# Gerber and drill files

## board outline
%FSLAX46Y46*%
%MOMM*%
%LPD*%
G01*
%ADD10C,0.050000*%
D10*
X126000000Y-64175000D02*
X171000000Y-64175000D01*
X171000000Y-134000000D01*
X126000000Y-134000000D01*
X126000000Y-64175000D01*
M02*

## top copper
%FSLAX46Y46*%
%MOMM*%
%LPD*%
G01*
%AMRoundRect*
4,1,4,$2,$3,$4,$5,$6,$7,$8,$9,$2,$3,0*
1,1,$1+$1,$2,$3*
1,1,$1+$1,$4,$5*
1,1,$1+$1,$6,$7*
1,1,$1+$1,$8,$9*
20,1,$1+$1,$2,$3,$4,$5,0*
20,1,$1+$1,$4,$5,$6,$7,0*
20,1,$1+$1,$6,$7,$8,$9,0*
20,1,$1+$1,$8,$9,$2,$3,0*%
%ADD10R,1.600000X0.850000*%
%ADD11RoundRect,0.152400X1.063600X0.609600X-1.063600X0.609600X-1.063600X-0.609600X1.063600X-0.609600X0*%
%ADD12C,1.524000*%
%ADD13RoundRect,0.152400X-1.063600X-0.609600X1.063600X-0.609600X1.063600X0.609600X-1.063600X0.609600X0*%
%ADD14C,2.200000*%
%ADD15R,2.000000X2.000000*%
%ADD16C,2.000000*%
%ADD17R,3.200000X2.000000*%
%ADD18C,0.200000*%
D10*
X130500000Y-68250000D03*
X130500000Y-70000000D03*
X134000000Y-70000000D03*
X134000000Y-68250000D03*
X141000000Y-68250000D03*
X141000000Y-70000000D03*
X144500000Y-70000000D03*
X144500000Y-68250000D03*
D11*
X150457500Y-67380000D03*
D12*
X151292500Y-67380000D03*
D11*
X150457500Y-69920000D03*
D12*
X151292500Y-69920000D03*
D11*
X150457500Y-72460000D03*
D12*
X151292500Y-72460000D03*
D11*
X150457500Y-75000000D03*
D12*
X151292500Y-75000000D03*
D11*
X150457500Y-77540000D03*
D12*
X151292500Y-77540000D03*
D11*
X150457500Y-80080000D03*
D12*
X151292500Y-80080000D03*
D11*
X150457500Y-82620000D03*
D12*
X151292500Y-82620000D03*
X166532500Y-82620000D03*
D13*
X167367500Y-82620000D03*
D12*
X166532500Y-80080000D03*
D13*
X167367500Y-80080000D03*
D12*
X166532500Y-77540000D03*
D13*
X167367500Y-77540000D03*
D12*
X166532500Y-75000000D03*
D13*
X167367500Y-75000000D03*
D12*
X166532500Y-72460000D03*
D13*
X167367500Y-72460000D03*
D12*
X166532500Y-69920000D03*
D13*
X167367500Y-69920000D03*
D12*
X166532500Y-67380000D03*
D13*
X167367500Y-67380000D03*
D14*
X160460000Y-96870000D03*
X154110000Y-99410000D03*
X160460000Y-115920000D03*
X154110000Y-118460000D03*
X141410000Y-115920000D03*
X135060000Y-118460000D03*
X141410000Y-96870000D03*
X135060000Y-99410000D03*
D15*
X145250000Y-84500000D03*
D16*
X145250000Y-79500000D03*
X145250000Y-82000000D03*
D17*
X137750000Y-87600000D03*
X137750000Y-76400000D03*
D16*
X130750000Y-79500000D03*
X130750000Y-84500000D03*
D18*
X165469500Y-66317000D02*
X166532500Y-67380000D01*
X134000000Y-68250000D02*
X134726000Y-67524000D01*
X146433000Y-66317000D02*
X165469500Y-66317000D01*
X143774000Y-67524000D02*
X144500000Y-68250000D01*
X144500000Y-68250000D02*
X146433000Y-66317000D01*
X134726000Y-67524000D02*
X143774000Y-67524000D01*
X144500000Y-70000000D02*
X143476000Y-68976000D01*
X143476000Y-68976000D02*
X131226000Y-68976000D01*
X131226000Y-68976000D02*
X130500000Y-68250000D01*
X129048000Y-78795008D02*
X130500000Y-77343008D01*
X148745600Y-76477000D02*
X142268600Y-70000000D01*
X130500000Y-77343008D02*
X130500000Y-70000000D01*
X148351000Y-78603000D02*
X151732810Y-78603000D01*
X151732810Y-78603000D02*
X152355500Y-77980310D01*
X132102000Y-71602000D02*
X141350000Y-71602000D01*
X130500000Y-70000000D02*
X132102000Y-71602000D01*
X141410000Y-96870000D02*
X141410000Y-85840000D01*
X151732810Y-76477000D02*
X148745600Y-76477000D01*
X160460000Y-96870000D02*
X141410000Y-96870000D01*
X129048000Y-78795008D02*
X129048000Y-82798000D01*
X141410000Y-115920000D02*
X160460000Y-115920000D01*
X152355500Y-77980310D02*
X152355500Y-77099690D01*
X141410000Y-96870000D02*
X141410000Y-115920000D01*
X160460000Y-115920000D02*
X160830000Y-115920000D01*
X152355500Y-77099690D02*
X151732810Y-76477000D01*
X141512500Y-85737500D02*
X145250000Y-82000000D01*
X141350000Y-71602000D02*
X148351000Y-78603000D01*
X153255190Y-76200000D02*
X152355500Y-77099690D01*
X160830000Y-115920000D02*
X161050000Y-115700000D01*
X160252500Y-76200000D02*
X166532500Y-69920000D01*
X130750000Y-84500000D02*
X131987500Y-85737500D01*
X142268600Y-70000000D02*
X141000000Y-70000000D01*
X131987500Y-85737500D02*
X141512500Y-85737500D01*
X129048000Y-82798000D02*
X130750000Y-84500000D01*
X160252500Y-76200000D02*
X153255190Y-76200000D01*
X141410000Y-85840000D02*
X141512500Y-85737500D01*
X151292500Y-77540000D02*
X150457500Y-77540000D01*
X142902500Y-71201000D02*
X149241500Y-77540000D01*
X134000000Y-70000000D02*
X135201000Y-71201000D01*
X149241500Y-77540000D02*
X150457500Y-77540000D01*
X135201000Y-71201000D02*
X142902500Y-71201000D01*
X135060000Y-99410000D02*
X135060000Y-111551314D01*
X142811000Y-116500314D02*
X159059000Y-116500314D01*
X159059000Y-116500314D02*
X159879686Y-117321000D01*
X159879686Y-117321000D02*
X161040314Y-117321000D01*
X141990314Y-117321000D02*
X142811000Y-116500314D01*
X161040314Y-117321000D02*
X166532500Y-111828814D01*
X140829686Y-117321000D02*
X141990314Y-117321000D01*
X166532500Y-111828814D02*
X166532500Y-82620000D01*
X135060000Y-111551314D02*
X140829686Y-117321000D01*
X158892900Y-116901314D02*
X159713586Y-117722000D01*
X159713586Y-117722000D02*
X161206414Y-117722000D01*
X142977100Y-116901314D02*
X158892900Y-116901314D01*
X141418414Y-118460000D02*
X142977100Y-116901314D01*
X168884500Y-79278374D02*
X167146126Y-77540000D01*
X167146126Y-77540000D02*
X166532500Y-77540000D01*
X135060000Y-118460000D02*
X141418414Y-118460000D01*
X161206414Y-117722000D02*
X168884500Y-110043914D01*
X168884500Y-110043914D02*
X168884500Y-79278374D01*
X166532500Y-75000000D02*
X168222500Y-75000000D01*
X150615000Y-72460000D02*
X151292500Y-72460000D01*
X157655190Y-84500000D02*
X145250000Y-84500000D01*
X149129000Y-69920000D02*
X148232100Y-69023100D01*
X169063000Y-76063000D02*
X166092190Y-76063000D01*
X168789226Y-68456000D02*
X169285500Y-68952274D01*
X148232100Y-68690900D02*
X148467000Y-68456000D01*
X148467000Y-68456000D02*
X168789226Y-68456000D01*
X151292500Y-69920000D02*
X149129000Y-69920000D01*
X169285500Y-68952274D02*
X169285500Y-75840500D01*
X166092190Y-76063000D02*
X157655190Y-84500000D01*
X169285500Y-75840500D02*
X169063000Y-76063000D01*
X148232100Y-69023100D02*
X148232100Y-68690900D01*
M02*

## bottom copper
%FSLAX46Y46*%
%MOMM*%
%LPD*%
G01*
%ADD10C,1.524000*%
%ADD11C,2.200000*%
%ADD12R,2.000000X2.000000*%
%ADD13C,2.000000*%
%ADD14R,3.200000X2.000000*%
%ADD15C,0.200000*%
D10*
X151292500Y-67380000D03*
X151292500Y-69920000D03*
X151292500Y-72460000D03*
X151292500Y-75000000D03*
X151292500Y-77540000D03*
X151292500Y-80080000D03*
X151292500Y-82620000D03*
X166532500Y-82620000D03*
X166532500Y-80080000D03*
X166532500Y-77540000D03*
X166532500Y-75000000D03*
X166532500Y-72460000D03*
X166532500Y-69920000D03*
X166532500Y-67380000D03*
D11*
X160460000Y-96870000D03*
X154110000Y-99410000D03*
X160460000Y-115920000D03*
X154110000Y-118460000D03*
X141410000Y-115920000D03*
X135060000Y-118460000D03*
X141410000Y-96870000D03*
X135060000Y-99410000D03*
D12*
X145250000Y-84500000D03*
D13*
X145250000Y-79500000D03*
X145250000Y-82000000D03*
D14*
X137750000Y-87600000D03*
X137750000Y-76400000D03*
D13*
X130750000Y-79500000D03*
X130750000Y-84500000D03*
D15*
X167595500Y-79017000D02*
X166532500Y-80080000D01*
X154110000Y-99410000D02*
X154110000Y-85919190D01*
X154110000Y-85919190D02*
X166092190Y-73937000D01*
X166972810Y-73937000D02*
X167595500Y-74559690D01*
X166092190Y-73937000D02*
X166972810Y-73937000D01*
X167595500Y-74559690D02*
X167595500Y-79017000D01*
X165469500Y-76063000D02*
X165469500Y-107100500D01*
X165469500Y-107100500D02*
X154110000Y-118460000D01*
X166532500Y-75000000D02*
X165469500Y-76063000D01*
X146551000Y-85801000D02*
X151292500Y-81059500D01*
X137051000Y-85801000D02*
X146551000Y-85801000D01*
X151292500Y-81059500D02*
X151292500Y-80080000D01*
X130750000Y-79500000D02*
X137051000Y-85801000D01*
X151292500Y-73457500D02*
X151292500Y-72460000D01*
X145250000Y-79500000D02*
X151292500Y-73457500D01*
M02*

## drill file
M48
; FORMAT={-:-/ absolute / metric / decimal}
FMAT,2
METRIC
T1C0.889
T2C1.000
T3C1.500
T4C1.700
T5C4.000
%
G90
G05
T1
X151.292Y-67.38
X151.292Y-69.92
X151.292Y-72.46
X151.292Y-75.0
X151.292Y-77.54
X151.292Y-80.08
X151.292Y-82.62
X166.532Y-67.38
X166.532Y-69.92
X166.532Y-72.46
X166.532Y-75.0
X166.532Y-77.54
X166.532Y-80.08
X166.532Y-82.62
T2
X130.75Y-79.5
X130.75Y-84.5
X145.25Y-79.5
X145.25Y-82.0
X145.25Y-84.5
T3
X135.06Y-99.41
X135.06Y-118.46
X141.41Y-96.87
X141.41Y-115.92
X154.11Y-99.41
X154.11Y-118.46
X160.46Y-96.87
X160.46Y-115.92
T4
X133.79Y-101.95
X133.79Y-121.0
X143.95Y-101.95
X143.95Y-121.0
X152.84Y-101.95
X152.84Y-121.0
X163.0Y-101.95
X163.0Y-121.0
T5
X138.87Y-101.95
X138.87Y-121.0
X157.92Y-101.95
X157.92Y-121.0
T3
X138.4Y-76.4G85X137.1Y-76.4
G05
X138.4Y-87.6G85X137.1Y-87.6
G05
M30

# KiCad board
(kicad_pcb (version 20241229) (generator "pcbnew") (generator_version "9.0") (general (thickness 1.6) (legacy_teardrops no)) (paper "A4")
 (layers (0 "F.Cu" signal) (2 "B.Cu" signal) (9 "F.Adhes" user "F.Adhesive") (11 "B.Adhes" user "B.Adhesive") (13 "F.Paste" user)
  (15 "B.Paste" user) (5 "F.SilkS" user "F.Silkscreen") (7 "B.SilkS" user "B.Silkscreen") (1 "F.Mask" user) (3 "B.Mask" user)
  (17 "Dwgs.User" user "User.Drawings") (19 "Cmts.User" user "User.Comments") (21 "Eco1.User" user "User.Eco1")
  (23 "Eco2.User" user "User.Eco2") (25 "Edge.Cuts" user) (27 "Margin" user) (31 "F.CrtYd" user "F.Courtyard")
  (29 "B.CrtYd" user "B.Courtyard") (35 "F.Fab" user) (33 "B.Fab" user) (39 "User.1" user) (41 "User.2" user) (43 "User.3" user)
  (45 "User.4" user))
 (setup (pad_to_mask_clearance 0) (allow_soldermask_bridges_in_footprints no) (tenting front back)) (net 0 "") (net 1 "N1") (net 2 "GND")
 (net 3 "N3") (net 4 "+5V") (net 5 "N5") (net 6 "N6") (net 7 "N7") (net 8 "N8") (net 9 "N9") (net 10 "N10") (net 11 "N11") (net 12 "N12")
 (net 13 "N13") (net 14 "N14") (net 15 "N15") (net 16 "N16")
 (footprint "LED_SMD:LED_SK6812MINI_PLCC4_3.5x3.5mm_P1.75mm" (layer "F.Cu") (at 132.25 69.125)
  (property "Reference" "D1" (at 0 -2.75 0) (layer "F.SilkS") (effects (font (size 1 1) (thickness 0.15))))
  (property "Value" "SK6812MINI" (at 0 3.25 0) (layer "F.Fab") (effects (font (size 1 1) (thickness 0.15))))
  (pad "1" smd rect (at -1.75 -0.875) (size 1.6 0.85) (layers "F.Cu" "F.Mask" "F.Paste") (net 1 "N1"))
  (pad "2" smd rect (at -1.75 0.875) (size 1.6 0.85) (layers "F.Cu" "F.Mask" "F.Paste") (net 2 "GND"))
  (pad "3" smd rect (at 1.75 0.875) (size 1.6 0.85) (layers "F.Cu" "F.Mask" "F.Paste") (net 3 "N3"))
  (pad "4" smd rect (at 1.75 -0.875) (size 1.6 0.85) (layers "F.Cu" "F.Mask" "F.Paste") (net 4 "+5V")))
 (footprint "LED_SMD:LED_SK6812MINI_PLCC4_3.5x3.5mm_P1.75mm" (layer "F.Cu") (at 142.75 69.125)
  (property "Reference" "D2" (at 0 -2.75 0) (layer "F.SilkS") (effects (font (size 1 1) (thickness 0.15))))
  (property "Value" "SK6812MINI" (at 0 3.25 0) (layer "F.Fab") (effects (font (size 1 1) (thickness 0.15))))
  (pad "1" smd rect (at -1.75 -0.875) (size 1.6 0.85) (layers "F.Cu" "F.Mask" "F.Paste") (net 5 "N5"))
  (pad "2" smd rect (at -1.75 0.875) (size 1.6 0.85) (layers "F.Cu" "F.Mask" "F.Paste") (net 2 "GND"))
  (pad "3" smd rect (at 1.75 0.875) (size 1.6 0.85) (layers "F.Cu" "F.Mask" "F.Paste") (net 1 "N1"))
  (pad "4" smd rect (at 1.75 -0.875) (size 1.6 0.85) (layers "F.Cu" "F.Mask" "F.Paste") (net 4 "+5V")))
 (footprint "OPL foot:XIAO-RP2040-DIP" (layer "F.Cu") (at 158.9125 75)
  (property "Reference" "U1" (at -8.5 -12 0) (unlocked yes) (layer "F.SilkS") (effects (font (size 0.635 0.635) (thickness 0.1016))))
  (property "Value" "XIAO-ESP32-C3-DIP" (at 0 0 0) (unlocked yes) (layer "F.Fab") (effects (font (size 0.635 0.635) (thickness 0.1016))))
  (pad "1" smd roundrect (at -8.455 -7.62 180) (size 2.432 1.524) (layers "F.Cu" "F.Mask") (roundrect_rratio 0.1) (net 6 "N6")
   (thermal_bridge_angle 45))
  (pad "1" thru_hole circle (at -7.62 -7.62 180) (size 1.524 1.524) (drill 0.889) (layers "*.Cu" "*.Mask") (remove_unused_layers no)
   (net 6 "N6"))
  (pad "2" smd roundrect (at -8.455 -5.08 180) (size 2.432 1.524) (layers "F.Cu" "F.Mask") (roundrect_rratio 0.1) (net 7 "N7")
   (thermal_bridge_angle 45))
  (pad "2" thru_hole circle (at -7.62 -5.08 180) (size 1.524 1.524) (drill 0.889) (layers "*.Cu" "*.Mask") (remove_unused_layers no)
   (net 7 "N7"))
  (pad "3" smd roundrect (at -8.455 -2.54 180) (size 2.432 1.524) (layers "F.Cu" "F.Mask") (roundrect_rratio 0.1) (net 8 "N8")
   (thermal_bridge_angle 45))
  (pad "3" thru_hole circle (at -7.62 -2.54 180) (size 1.524 1.524) (drill 0.889) (layers "*.Cu" "*.Mask") (remove_unused_layers no)
   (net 8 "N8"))
  (pad "4" smd roundrect (at -8.455 0 180) (size 2.432 1.524) (layers "F.Cu" "F.Mask") (roundrect_rratio 0.1) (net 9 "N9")
   (thermal_bridge_angle 45))
  (pad "4" thru_hole circle (at -7.62 0 180) (size 1.524 1.524) (drill 0.889) (layers "*.Cu" "*.Mask") (remove_unused_layers no)
   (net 9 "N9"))
  (pad "5" smd roundrect (at -8.455 2.54 180) (size 2.432 1.524) (layers "F.Cu" "F.Mask") (roundrect_rratio 0.1) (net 3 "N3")
   (thermal_bridge_angle 45))
  (pad "5" thru_hole circle (at -7.62 2.54 180) (size 1.524 1.524) (drill 0.889) (layers "*.Cu" "*.Mask") (remove_unused_layers no)
   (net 3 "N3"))
  (pad "6" smd roundrect (at -8.455 5.08 180) (size 2.432 1.524) (layers "F.Cu" "F.Mask") (roundrect_rratio 0.1) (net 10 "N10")
   (thermal_bridge_angle 45))
  (pad "6" thru_hole circle (at -7.62 5.08 180) (size 1.524 1.524) (drill 0.889) (layers "*.Cu" "*.Mask") (remove_unused_layers no)
   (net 10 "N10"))
  (pad "7" smd roundrect (at -8.455 7.62 180) (size 2.432 1.524) (layers "F.Cu" "F.Mask") (roundrect_rratio 0.1) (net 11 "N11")
   (thermal_bridge_angle 45))
  (pad "7" thru_hole circle (at -7.62 7.62 180) (size 1.524 1.524) (drill 0.889) (layers "*.Cu" "*.Mask") (remove_unused_layers no)
   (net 11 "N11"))
  (pad "8" thru_hole circle (at 7.62 7.62) (size 1.524 1.524) (drill 0.889) (layers "*.Cu" "*.Mask") (remove_unused_layers no)
   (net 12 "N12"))
  (pad "8" smd roundrect (at 8.455 7.62) (size 2.432 1.524) (layers "F.Cu" "F.Mask") (roundrect_rratio 0.1) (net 12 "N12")
   (thermal_bridge_angle 45))
  (pad "9" thru_hole circle (at 7.62 5.08) (size 1.524 1.524) (drill 0.889) (layers "*.Cu" "*.Mask") (remove_unused_layers no)
   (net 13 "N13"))
  (pad "9" smd roundrect (at 8.455 5.08) (size 2.432 1.524) (layers "F.Cu" "F.Mask") (roundrect_rratio 0.1) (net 13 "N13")
   (thermal_bridge_angle 45))
  (pad "10" thru_hole circle (at 7.62 2.54) (size 1.524 1.524) (drill 0.889) (layers "*.Cu" "*.Mask") (remove_unused_layers no)
   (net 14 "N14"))
  (pad "10" smd roundrect (at 8.455 2.54) (size 2.432 1.524) (layers "F.Cu" "F.Mask") (roundrect_rratio 0.1) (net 14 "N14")
   (thermal_bridge_angle 45))
  (pad "11" thru_hole circle (at 7.62 0) (size 1.524 1.524) (drill 0.889) (layers "*.Cu" "*.Mask") (remove_unused_layers no) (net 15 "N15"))
  (pad "11" smd roundrect (at 8.455 0) (size 2.432 1.524) (layers "F.Cu" "F.Mask") (roundrect_rratio 0.1) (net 15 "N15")
   (thermal_bridge_angle 45))
  (pad "12" thru_hole circle (at 7.62 -2.54) (size 1.524 1.524) (drill 0.889) (layers "*.Cu" "*.Mask") (remove_unused_layers no)
   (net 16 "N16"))
  (pad "12" smd roundrect (at 8.455 -2.54) (size 2.432 1.524) (layers "F.Cu" "F.Mask") (roundrect_rratio 0.1) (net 16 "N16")
   (thermal_bridge_angle 45))
  (pad "13" thru_hole circle (at 7.62 -5.08) (size 1.524 1.524) (drill 0.889) (layers "*.Cu" "*.Mask") (remove_unused_layers no)
   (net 2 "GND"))
  (pad "13" smd roundrect (at 8.455 -5.08) (size 2.432 1.524) (layers "F.Cu" "F.Mask") (roundrect_rratio 0.1) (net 2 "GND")
   (thermal_bridge_angle 45))
  (pad "14" thru_hole circle (at 7.62 -7.62) (size 1.524 1.524) (drill 0.889) (layers "*.Cu" "*.Mask") (remove_unused_layers no)
   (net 4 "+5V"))
  (pad "14" smd roundrect (at 8.455 -7.62) (size 2.432 1.524) (layers "F.Cu" "F.Mask") (roundrect_rratio 0.1) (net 4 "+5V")
   (thermal_bridge_angle 45)))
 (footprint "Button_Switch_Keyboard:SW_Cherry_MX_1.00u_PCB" (layer "F.Cu") (at 160.46 96.87)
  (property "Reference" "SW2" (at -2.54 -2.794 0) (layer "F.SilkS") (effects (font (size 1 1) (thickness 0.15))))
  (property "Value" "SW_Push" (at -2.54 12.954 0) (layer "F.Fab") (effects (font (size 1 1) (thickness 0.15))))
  (pad "" np_thru_hole circle (at -7.62 5.08) (size 1.7 1.7) (drill 1.7) (layers "*.Cu" "*.Mask"))
  (pad "" np_thru_hole circle (at -2.54 5.08) (size 4 4) (drill 4) (layers "*.Cu" "*.Mask"))
  (pad "" np_thru_hole circle (at 2.54 5.08) (size 1.7 1.7) (drill 1.7) (layers "*.Cu" "*.Mask"))
  (pad "1" thru_hole circle (at 0 0) (size 2.2 2.2) (drill 1.5) (layers "*.Cu" "*.Mask") (remove_unused_layers no) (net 2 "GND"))
  (pad "2" thru_hole circle (at -6.35 2.54) (size 2.2 2.2) (drill 1.5) (layers "*.Cu" "*.Mask") (remove_unused_layers no) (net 13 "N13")))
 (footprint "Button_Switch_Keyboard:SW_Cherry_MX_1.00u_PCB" (layer "F.Cu") (at 160.46 115.92)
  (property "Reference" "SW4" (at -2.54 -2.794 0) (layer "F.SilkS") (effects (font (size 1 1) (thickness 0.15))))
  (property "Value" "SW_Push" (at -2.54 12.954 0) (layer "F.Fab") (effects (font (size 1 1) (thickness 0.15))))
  (pad "" np_thru_hole circle (at -7.62 5.08) (size 1.7 1.7) (drill 1.7) (layers "*.Cu" "*.Mask"))
  (pad "" np_thru_hole circle (at -2.54 5.08) (size 4 4) (drill 4) (layers "*.Cu" "*.Mask"))
  (pad "" np_thru_hole circle (at 2.54 5.08) (size 1.7 1.7) (drill 1.7) (layers "*.Cu" "*.Mask"))
  (pad "1" thru_hole circle (at 0 0) (size 2.2 2.2) (drill 1.5) (layers "*.Cu" "*.Mask") (remove_unused_layers no) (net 2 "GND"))
  (pad "2" thru_hole circle (at -6.35 2.54) (size 2.2 2.2) (drill 1.5) (layers "*.Cu" "*.Mask") (remove_unused_layers no) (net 15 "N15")))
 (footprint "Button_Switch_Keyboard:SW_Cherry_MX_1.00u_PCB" (layer "F.Cu") (at 141.41 115.92)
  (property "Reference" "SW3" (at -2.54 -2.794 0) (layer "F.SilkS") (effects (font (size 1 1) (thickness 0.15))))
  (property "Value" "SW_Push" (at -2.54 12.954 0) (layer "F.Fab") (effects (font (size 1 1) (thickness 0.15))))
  (pad "" np_thru_hole circle (at -7.62 5.08) (size 1.7 1.7) (drill 1.7) (layers "*.Cu" "*.Mask"))
  (pad "" np_thru_hole circle (at -2.54 5.08) (size 4 4) (drill 4) (layers "*.Cu" "*.Mask"))
  (pad "" np_thru_hole circle (at 2.54 5.08) (size 1.7 1.7) (drill 1.7) (layers "*.Cu" "*.Mask"))
  (pad "1" thru_hole circle (at 0 0) (size 2.2 2.2) (drill 1.5) (layers "*.Cu" "*.Mask") (remove_unused_layers no) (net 2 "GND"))
  (pad "2" thru_hole circle (at -6.35 2.54) (size 2.2 2.2) (drill 1.5) (layers "*.Cu" "*.Mask") (remove_unused_layers no) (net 14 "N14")))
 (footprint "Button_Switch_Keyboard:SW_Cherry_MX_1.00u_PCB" (layer "F.Cu") (at 141.41 96.87)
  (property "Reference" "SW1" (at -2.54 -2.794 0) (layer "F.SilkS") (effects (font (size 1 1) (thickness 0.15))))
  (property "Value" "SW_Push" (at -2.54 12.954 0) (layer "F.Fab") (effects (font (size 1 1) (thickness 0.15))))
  (pad "" np_thru_hole circle (at -7.62 5.08) (size 1.7 1.7) (drill 1.7) (layers "*.Cu" "*.Mask"))
  (pad "" np_thru_hole circle (at -2.54 5.08) (size 4 4) (drill 4) (layers "*.Cu" "*.Mask"))
  (pad "" np_thru_hole circle (at 2.54 5.08) (size 1.7 1.7) (drill 1.7) (layers "*.Cu" "*.Mask"))
  (pad "1" thru_hole circle (at 0 0) (size 2.2 2.2) (drill 1.5) (layers "*.Cu" "*.Mask") (remove_unused_layers no) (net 2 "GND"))
  (pad "2" thru_hole circle (at -6.35 2.54) (size 2.2 2.2) (drill 1.5) (layers "*.Cu" "*.Mask") (remove_unused_layers no) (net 12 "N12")))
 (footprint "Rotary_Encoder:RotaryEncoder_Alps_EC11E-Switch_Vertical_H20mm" (layer "F.Cu") (at 145.25 84.5 180)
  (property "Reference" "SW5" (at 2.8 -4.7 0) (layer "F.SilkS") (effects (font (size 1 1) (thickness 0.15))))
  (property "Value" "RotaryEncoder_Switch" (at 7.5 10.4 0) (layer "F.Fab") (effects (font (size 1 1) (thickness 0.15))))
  (pad "A" thru_hole rect (at 0 0 180) (size 2 2) (drill 1) (layers "*.Cu" "*.Mask") (remove_unused_layers no) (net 7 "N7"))
  (pad "B" thru_hole circle (at 0 5 180) (size 2 2) (drill 1) (layers "*.Cu" "*.Mask") (remove_unused_layers no) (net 8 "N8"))
  (pad "C" thru_hole circle (at 0 2.5 180) (size 2 2) (drill 1) (layers "*.Cu" "*.Mask") (remove_unused_layers no) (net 2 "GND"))
  (pad "MP" thru_hole rect (at 7.5 -3.1 180) (size 3.2 2) (drill oval 2.8 1.5) (layers "*.Cu" "*.Mask") (remove_unused_layers no))
  (pad "MP" thru_hole rect (at 7.5 8.1 180) (size 3.2 2) (drill oval 2.8 1.5) (layers "*.Cu" "*.Mask") (remove_unused_layers no))
  (pad "S1" thru_hole circle (at 14.5 5 180) (size 2 2) (drill 1) (layers "*.Cu" "*.Mask") (remove_unused_layers no) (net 10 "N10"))
  (pad "S2" thru_hole circle (at 14.5 0 180) (size 2 2) (drill 1) (layers "*.Cu" "*.Mask") (remove_unused_layers no) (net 2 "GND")))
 (gr_rect (start 126 64.175) (end 171 134) (stroke (width 0.05) (type default)) (fill no) (layer "Edge.Cuts"))
 (segment (start 165.4695 66.317) (end 166.5325 67.38) (width 0.2) (layer "F.Cu") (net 4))
 (segment (start 134 68.25) (end 134.726 67.524) (width 0.2) (layer "F.Cu") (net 4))
 (segment (start 146.433 66.317) (end 165.4695 66.317) (width 0.2) (layer "F.Cu") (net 4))
 (segment (start 143.774 67.524) (end 144.5 68.25) (width 0.2) (layer "F.Cu") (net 4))
 (segment (start 144.5 68.25) (end 146.433 66.317) (width 0.2) (layer "F.Cu") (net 4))
 (segment (start 134.726 67.524) (end 143.774 67.524) (width 0.2) (layer "F.Cu") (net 4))
 (segment (start 144.5 70) (end 143.476 68.976) (width 0.2) (layer "F.Cu") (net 1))
 (segment (start 143.476 68.976) (end 131.226 68.976) (width 0.2) (layer "F.Cu") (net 1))
 (segment (start 131.226 68.976) (end 130.5 68.25) (width 0.2) (layer "F.Cu") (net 1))
 (segment (start 129.048 78.795008) (end 130.5 77.343008) (width 0.2) (layer "F.Cu") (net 2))
 (segment (start 148.7456 76.477) (end 142.2686 70) (width 0.2) (layer "F.Cu") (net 2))
 (segment (start 130.5 77.343008) (end 130.5 70) (width 0.2) (layer "F.Cu") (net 2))
 (segment (start 148.351 78.603) (end 151.73281 78.603) (width 0.2) (layer "F.Cu") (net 2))
 (segment (start 151.73281 78.603) (end 152.3555 77.98031) (width 0.2) (layer "F.Cu") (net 2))
 (segment (start 132.102 71.602) (end 141.35 71.602) (width 0.2) (layer "F.Cu") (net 2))
 (segment (start 130.5 70) (end 132.102 71.602) (width 0.2) (layer "F.Cu") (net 2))
 (segment (start 141.41 96.87) (end 141.41 85.84) (width 0.2) (layer "F.Cu") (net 2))
 (segment (start 151.73281 76.477) (end 148.7456 76.477) (width 0.2) (layer "F.Cu") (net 2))
 (segment (start 160.46 96.87) (end 141.41 96.87) (width 0.2) (layer "F.Cu") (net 2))
 (segment (start 129.048 78.795008) (end 129.048 82.798) (width 0.2) (layer "F.Cu") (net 2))
 (segment (start 141.41 115.92) (end 160.46 115.92) (width 0.2) (layer "F.Cu") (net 2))
 (segment (start 152.3555 77.98031) (end 152.3555 77.09969) (width 0.2) (layer "F.Cu") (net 2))
 (segment (start 141.41 96.87) (end 141.41 115.92) (width 0.2) (layer "F.Cu") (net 2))
 (segment (start 160.46 115.92) (end 160.83 115.92) (width 0.2) (layer "F.Cu") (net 2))
 (segment (start 152.3555 77.09969) (end 151.73281 76.477) (width 0.2) (layer "F.Cu") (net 2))
 (segment (start 141.5125 85.7375) (end 145.25 82) (width 0.2) (layer "F.Cu") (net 2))
 (segment (start 141.35 71.602) (end 148.351 78.603) (width 0.2) (layer "F.Cu") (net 2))
 (segment (start 153.25519 76.2) (end 152.3555 77.09969) (width 0.2) (layer "F.Cu") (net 2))
 (segment (start 160.83 115.92) (end 161.05 115.7) (width 0.2) (layer "F.Cu") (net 2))
 (segment (start 160.2525 76.2) (end 166.5325 69.92) (width 0.2) (layer "F.Cu") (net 2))
 (segment (start 130.75 84.5) (end 131.9875 85.7375) (width 0.2) (layer "F.Cu") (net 2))
 (segment (start 142.2686 70) (end 141 70) (width 0.2) (layer "F.Cu") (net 2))
 (segment (start 131.9875 85.7375) (end 141.5125 85.7375) (width 0.2) (layer "F.Cu") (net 2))
 (segment (start 129.048 82.798) (end 130.75 84.5) (width 0.2) (layer "F.Cu") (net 2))
 (segment (start 160.2525 76.2) (end 153.25519 76.2) (width 0.2) (layer "F.Cu") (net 2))
 (segment (start 141.41 85.84) (end 141.5125 85.7375) (width 0.2) (layer "F.Cu") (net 2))
 (segment (start 151.2925 77.54) (end 150.4575 77.54) (width 0.2) (layer "F.Cu") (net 3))
 (segment (start 142.9025 71.201) (end 149.2415 77.54) (width 0.2) (layer "F.Cu") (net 3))
 (segment (start 134 70) (end 135.201 71.201) (width 0.2) (layer "F.Cu") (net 3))
 (segment (start 149.2415 77.54) (end 150.4575 77.54) (width 0.2) (layer "F.Cu") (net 3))
 (segment (start 135.201 71.201) (end 142.9025 71.201) (width 0.2) (layer "F.Cu") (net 3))
 (segment (start 135.06 99.41) (end 135.06 111.551314) (width 0.2) (layer "F.Cu") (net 12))
 (segment (start 142.811 116.500314) (end 159.059 116.500314) (width 0.2) (layer "F.Cu") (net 12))
 (segment (start 159.059 116.500314) (end 159.879686 117.321) (width 0.2) (layer "F.Cu") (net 12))
 (segment (start 159.879686 117.321) (end 161.040314 117.321) (width 0.2) (layer "F.Cu") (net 12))
 (segment (start 141.990314 117.321) (end 142.811 116.500314) (width 0.2) (layer "F.Cu") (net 12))
 (segment (start 161.040314 117.321) (end 166.5325 111.828814) (width 0.2) (layer "F.Cu") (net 12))
 (segment (start 140.829686 117.321) (end 141.990314 117.321) (width 0.2) (layer "F.Cu") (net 12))
 (segment (start 166.5325 111.828814) (end 166.5325 82.62) (width 0.2) (layer "F.Cu") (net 12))
 (segment (start 135.06 111.551314) (end 140.829686 117.321) (width 0.2) (layer "F.Cu") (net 12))
 (segment (start 167.5955 79.017) (end 166.5325 80.08) (width 0.2) (layer "B.Cu") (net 13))
 (segment (start 154.11 99.41) (end 154.11 85.91919) (width 0.2) (layer "B.Cu") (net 13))
 (segment (start 154.11 85.91919) (end 166.09219 73.937) (width 0.2) (layer "B.Cu") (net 13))
 (segment (start 166.97281 73.937) (end 167.5955 74.55969) (width 0.2) (layer "B.Cu") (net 13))
 (segment (start 166.09219 73.937) (end 166.97281 73.937) (width 0.2) (layer "B.Cu") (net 13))
 (segment (start 167.5955 74.55969) (end 167.5955 79.017) (width 0.2) (layer "B.Cu") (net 13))
 (segment (start 158.8929 116.901314) (end 159.713586 117.722) (width 0.2) (layer "F.Cu") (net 14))
 (segment (start 159.713586 117.722) (end 161.206414 117.722) (width 0.2) (layer "F.Cu") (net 14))
 (segment (start 142.9771 116.901314) (end 158.8929 116.901314) (width 0.2) (layer "F.Cu") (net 14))
 (segment (start 141.418414 118.46) (end 142.9771 116.901314) (width 0.2) (layer "F.Cu") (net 14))
 (segment (start 168.8845 79.278374) (end 167.146126 77.54) (width 0.2) (layer "F.Cu") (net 14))
 (segment (start 167.146126 77.54) (end 166.5325 77.54) (width 0.2) (layer "F.Cu") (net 14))
 (segment (start 135.06 118.46) (end 141.418414 118.46) (width 0.2) (layer "F.Cu") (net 14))
 (segment (start 161.206414 117.722) (end 168.8845 110.043914) (width 0.2) (layer "F.Cu") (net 14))
 (segment (start 168.8845 110.043914) (end 168.8845 79.278374) (width 0.2) (layer "F.Cu") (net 14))
 (segment (start 166.5325 75) (end 168.2225 75) (width 0.2) (layer "F.Cu") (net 15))
 (segment (start 165.4695 76.063) (end 165.4695 107.1005) (width 0.2) (layer "B.Cu") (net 15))
 (segment (start 165.4695 107.1005) (end 154.11 118.46) (width 0.2) (layer "B.Cu") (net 15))
 (segment (start 166.5325 75) (end 165.4695 76.063) (width 0.2) (layer "B.Cu") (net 15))
 (segment (start 146.551 85.801) (end 151.2925 81.0595) (width 0.2) (layer "B.Cu") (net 10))
 (segment (start 137.051 85.801) (end 146.551 85.801) (width 0.2) (layer "B.Cu") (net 10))
 (segment (start 151.2925 81.0595) (end 151.2925 80.08) (width 0.2) (layer "B.Cu") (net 10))
 (segment (start 130.75 79.5) (end 137.051 85.801) (width 0.2) (layer "B.Cu") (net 10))
 (segment (start 150.615 72.46) (end 151.2925 72.46) (width 0.2) (layer "F.Cu") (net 8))
 (segment (start 151.2925 73.4575) (end 151.2925 72.46) (width 0.2) (layer "B.Cu") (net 8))
 (segment (start 145.25 79.5) (end 151.2925 73.4575) (width 0.2) (layer "B.Cu") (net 8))
 (segment (start 157.65519 84.5) (end 145.25 84.5) (width 0.2) (layer "F.Cu") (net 7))
 (segment (start 149.129 69.92) (end 148.2321 69.0231) (width 0.2) (layer "F.Cu") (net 7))
 (segment (start 169.063 76.063) (end 166.09219 76.063) (width 0.2) (layer "F.Cu") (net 7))
 (segment (start 168.789226 68.456) (end 169.2855 68.952274) (width 0.2) (layer "F.Cu") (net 7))
 (segment (start 148.2321 68.6909) (end 148.467 68.456) (width 0.2) (layer "F.Cu") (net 7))
 (segment (start 148.467 68.456) (end 168.789226 68.456) (width 0.2) (layer "F.Cu") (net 7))
 (segment (start 151.2925 69.92) (end 149.129 69.92) (width 0.2) (layer "F.Cu") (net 7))
 (segment (start 169.2855 68.952274) (end 169.2855 75.8405) (width 0.2) (layer "F.Cu") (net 7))
 (segment (start 166.09219 76.063) (end 157.65519 84.5) (width 0.2) (layer "F.Cu") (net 7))
 (segment (start 169.2855 75.8405) (end 169.063 76.063) (width 0.2) (layer "F.Cu") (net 7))
 (segment (start 148.2321 69.0231) (end 148.2321 68.6909) (width 0.2) (layer "F.Cu") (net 7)))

